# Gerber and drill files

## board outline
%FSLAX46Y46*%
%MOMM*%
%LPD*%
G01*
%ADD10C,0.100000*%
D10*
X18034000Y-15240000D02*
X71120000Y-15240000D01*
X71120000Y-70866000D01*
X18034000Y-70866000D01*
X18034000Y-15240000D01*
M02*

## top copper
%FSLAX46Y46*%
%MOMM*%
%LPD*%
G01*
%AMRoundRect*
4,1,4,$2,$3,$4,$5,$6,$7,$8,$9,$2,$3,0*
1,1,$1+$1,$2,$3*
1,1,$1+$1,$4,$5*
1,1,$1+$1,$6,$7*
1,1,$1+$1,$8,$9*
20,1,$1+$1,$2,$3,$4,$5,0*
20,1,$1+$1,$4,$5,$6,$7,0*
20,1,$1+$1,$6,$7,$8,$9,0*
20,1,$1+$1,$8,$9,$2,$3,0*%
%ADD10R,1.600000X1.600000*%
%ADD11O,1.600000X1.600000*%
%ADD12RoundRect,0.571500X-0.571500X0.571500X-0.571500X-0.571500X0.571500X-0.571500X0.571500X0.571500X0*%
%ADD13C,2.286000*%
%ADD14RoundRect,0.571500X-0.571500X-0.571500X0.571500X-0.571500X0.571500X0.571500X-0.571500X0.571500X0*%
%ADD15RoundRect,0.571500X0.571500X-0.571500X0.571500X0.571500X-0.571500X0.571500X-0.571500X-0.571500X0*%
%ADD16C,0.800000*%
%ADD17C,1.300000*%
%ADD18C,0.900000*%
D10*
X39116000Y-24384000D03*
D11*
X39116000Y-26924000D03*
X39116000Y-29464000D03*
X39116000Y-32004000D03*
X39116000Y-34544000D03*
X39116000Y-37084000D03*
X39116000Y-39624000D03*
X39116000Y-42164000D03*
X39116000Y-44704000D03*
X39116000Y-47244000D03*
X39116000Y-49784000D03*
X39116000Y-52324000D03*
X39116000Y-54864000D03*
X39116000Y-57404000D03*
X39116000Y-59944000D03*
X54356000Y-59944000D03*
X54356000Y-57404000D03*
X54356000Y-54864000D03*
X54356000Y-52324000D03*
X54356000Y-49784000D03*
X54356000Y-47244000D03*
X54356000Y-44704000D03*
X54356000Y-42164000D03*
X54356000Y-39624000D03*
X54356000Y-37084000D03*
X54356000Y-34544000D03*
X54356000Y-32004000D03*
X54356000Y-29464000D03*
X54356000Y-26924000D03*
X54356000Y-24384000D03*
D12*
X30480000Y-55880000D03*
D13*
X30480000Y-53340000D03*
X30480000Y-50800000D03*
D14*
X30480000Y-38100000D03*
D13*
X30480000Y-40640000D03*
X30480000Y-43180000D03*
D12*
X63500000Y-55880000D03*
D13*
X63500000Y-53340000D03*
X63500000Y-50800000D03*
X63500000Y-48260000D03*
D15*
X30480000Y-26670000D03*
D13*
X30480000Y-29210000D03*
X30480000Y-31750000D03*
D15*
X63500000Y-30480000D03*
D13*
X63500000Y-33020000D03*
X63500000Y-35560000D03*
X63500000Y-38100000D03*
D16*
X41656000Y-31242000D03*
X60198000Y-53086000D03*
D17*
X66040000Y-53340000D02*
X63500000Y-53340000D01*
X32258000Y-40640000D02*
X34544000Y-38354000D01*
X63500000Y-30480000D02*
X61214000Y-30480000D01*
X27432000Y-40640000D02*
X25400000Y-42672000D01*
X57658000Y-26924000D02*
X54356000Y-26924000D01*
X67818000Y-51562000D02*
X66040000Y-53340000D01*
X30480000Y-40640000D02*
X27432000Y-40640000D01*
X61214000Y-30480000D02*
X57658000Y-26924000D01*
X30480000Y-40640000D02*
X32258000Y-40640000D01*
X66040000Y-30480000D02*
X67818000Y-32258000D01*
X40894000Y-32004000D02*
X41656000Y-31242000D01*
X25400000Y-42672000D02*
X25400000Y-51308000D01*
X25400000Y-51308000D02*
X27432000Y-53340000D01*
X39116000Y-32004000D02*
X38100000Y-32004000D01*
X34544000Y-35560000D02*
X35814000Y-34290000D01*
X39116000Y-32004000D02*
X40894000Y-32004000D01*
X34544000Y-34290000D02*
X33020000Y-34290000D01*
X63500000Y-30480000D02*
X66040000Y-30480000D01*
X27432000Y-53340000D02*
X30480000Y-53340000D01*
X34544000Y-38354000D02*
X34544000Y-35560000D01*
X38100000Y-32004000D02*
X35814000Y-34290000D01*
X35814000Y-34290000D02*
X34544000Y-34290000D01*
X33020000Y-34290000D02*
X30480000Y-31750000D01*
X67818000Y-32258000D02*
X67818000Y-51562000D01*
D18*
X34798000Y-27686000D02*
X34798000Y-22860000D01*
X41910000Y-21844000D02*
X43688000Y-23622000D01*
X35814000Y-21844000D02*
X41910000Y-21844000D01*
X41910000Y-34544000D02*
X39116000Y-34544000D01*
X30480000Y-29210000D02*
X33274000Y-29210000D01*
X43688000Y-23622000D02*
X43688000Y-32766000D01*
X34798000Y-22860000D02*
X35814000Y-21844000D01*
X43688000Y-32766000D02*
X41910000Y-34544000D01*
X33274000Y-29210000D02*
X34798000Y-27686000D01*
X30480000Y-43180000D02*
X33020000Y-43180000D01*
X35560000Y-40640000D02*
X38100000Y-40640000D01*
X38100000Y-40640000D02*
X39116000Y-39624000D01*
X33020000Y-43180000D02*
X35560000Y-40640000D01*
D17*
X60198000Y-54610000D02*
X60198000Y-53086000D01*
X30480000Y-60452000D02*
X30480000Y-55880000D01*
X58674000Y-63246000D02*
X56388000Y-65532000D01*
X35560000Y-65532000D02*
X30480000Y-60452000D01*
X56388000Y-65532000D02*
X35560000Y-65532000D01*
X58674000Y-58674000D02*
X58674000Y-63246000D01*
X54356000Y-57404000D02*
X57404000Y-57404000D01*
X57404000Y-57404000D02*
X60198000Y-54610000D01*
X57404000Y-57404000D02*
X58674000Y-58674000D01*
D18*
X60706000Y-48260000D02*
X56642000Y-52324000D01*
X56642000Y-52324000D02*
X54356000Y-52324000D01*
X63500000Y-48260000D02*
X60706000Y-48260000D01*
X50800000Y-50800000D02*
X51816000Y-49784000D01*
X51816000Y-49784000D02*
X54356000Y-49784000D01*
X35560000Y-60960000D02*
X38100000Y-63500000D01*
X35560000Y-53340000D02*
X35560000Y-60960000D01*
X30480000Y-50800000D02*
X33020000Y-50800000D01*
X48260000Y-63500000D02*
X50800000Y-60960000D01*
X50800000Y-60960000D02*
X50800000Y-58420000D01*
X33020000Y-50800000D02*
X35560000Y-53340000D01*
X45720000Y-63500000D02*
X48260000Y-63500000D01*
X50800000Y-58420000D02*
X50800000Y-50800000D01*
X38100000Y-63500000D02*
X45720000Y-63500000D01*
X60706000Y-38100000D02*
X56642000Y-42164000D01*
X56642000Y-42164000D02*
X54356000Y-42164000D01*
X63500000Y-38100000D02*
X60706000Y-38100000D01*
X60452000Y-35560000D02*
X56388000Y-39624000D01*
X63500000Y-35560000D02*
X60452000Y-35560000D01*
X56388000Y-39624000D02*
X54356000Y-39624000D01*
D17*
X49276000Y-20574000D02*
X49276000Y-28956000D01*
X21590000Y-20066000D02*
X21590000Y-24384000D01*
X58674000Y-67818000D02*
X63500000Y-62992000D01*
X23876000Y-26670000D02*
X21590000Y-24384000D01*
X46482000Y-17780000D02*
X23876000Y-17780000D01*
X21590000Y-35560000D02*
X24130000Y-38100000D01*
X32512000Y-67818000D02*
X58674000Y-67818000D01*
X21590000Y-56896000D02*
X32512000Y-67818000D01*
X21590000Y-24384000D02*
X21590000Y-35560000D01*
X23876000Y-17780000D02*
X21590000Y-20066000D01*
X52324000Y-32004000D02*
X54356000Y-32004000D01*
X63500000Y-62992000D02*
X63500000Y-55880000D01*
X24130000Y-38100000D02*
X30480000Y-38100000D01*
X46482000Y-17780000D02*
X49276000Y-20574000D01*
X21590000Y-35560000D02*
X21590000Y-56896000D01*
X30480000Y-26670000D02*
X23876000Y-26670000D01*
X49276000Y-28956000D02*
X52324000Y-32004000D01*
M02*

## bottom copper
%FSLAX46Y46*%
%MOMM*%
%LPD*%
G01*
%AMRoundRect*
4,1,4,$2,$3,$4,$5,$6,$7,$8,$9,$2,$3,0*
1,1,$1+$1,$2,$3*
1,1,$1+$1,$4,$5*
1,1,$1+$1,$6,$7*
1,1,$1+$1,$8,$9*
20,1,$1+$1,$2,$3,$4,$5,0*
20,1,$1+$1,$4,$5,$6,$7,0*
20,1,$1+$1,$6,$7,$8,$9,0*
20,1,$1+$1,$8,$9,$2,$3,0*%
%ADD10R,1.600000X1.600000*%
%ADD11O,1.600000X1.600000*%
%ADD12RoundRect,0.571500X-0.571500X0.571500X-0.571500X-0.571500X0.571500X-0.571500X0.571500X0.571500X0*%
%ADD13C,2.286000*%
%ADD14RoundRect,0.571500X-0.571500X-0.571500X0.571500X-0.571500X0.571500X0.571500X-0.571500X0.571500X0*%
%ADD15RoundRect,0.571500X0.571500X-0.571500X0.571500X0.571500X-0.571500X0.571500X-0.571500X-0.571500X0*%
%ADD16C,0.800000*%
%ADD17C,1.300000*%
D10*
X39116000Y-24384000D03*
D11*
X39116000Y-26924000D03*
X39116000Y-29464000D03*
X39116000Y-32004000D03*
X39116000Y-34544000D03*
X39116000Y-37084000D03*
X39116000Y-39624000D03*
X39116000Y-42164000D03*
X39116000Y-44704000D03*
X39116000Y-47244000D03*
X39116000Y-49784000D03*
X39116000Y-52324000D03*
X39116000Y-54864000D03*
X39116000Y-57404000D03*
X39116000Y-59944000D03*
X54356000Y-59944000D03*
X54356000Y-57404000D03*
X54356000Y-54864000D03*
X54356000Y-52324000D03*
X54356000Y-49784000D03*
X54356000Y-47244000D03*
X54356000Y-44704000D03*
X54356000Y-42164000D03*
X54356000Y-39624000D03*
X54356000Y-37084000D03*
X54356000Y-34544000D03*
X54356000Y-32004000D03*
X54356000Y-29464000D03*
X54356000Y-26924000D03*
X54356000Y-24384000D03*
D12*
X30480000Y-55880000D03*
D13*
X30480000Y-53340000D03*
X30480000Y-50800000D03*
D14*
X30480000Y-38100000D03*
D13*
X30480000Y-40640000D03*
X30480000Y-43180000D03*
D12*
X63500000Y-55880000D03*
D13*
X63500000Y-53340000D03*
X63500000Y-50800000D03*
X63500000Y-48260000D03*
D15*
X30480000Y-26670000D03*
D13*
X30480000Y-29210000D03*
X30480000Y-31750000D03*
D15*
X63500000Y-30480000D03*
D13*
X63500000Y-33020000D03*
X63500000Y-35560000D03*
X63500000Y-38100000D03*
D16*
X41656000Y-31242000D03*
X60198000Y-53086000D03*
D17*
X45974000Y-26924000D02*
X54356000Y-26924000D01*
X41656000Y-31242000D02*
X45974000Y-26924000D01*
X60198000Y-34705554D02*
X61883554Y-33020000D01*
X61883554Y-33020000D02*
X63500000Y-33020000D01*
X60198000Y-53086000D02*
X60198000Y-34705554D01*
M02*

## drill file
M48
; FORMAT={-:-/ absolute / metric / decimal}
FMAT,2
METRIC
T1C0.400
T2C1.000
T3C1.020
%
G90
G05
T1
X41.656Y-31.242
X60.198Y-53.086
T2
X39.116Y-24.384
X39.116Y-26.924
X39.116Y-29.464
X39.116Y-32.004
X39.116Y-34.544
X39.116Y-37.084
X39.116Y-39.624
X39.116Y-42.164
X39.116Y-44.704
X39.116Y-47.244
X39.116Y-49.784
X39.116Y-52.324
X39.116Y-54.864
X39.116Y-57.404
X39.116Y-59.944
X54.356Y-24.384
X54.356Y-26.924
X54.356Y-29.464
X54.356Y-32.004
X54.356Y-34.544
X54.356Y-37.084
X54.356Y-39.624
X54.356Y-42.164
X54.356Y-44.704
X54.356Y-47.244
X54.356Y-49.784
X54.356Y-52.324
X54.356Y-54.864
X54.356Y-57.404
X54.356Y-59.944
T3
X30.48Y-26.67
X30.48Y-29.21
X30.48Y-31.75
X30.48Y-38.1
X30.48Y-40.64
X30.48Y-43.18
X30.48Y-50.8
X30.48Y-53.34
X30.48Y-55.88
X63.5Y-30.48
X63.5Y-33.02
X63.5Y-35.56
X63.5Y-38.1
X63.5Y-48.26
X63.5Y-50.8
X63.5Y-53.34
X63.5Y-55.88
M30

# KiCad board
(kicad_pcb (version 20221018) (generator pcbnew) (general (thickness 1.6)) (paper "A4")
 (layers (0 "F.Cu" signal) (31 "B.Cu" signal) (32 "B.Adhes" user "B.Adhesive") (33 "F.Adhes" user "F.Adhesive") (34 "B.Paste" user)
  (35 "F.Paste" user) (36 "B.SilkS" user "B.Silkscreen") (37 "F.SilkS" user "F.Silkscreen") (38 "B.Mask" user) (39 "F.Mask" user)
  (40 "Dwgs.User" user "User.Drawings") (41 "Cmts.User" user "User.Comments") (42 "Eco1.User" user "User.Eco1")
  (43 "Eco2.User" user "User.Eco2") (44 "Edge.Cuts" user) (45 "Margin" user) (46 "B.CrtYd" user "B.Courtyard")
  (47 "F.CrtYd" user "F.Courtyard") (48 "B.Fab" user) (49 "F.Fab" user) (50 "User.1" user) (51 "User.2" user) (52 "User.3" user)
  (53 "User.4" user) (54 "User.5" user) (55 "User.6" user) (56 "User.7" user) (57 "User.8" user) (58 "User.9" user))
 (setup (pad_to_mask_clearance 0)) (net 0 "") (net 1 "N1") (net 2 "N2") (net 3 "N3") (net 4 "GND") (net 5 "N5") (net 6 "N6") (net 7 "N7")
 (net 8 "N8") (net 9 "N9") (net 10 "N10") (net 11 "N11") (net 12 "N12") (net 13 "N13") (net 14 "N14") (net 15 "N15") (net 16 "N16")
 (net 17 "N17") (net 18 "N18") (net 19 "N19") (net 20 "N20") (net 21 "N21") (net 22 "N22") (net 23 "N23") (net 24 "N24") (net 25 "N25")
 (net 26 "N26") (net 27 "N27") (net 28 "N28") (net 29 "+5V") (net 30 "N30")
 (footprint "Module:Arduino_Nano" (layer "F.Cu") (at 39.116 24.384)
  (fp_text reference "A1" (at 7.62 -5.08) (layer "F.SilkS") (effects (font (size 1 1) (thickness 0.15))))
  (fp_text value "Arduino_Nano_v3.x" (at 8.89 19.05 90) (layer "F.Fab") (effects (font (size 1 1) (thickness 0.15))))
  (pad "1" thru_hole rect (at 0 0) (size 1.6 1.6) (drill 1) (layers "*.Cu" "*.Mask") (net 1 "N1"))
  (pad "2" thru_hole oval (at 0 2.54) (size 1.6 1.6) (drill 1) (layers "*.Cu" "*.Mask") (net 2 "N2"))
  (pad "3" thru_hole oval (at 0 5.08) (size 1.6 1.6) (drill 1) (layers "*.Cu" "*.Mask") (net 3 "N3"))
  (pad "4" thru_hole oval (at 0 7.62) (size 1.6 1.6) (drill 1) (layers "*.Cu" "*.Mask") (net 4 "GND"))
  (pad "5" thru_hole oval (at 0 10.16) (size 1.6 1.6) (drill 1) (layers "*.Cu" "*.Mask") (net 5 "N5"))
  (pad "6" thru_hole oval (at 0 12.7) (size 1.6 1.6) (drill 1) (layers "*.Cu" "*.Mask") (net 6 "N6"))
  (pad "7" thru_hole oval (at 0 15.24) (size 1.6 1.6) (drill 1) (layers "*.Cu" "*.Mask") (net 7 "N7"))
  (pad "8" thru_hole oval (at 0 17.78) (size 1.6 1.6) (drill 1) (layers "*.Cu" "*.Mask") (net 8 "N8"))
  (pad "9" thru_hole oval (at 0 20.32) (size 1.6 1.6) (drill 1) (layers "*.Cu" "*.Mask") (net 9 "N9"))
  (pad "10" thru_hole oval (at 0 22.86) (size 1.6 1.6) (drill 1) (layers "*.Cu" "*.Mask") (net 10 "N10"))
  (pad "11" thru_hole oval (at 0 25.4) (size 1.6 1.6) (drill 1) (layers "*.Cu" "*.Mask") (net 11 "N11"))
  (pad "12" thru_hole oval (at 0 27.94) (size 1.6 1.6) (drill 1) (layers "*.Cu" "*.Mask") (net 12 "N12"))
  (pad "13" thru_hole oval (at 0 30.48) (size 1.6 1.6) (drill 1) (layers "*.Cu" "*.Mask") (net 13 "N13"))
  (pad "14" thru_hole oval (at 0 33.02) (size 1.6 1.6) (drill 1) (layers "*.Cu" "*.Mask") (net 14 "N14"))
  (pad "15" thru_hole oval (at 0 35.56) (size 1.6 1.6) (drill 1) (layers "*.Cu" "*.Mask") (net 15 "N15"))
  (pad "16" thru_hole oval (at 15.24 35.56) (size 1.6 1.6) (drill 1) (layers "*.Cu" "*.Mask") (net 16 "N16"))
  (pad "17" thru_hole oval (at 15.24 33.02) (size 1.6 1.6) (drill 1) (layers "*.Cu" "*.Mask") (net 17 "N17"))
  (pad "18" thru_hole oval (at 15.24 30.48) (size 1.6 1.6) (drill 1) (layers "*.Cu" "*.Mask") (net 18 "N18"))
  (pad "19" thru_hole oval (at 15.24 27.94) (size 1.6 1.6) (drill 1) (layers "*.Cu" "*.Mask") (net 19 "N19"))
  (pad "20" thru_hole oval (at 15.24 25.4) (size 1.6 1.6) (drill 1) (layers "*.Cu" "*.Mask") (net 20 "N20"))
  (pad "21" thru_hole oval (at 15.24 22.86) (size 1.6 1.6) (drill 1) (layers "*.Cu" "*.Mask") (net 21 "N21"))
  (pad "22" thru_hole oval (at 15.24 20.32) (size 1.6 1.6) (drill 1) (layers "*.Cu" "*.Mask") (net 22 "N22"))
  (pad "23" thru_hole oval (at 15.24 17.78) (size 1.6 1.6) (drill 1) (layers "*.Cu" "*.Mask") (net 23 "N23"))
  (pad "24" thru_hole oval (at 15.24 15.24) (size 1.6 1.6) (drill 1) (layers "*.Cu" "*.Mask") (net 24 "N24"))
  (pad "25" thru_hole oval (at 15.24 12.7) (size 1.6 1.6) (drill 1) (layers "*.Cu" "*.Mask") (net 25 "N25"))
  (pad "26" thru_hole oval (at 15.24 10.16) (size 1.6 1.6) (drill 1) (layers "*.Cu" "*.Mask") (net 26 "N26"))
  (pad "27" thru_hole oval (at 15.24 7.62) (size 1.6 1.6) (drill 1) (layers "*.Cu" "*.Mask") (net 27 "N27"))
  (pad "28" thru_hole oval (at 15.24 5.08) (size 1.6 1.6) (drill 1) (layers "*.Cu" "*.Mask") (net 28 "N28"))
  (pad "29" thru_hole oval (at 15.24 2.54) (size 1.6 1.6) (drill 1) (layers "*.Cu" "*.Mask") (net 4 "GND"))
  (pad "30" thru_hole oval (at 15.24 0) (size 1.6 1.6) (drill 1) (layers "*.Cu" "*.Mask") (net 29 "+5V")))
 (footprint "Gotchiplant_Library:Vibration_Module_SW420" (layer "F.Cu") (at 30.48 53.34 180)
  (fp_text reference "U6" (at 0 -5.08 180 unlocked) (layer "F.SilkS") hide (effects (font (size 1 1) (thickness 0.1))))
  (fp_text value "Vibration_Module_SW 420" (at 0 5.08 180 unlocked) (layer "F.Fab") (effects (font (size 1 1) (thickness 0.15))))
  (pad "1" thru_hole roundrect (at 0 -2.54 270) (size 2.286 2.286) (drill 1.02) (layers "*.Cu" "*.Mask") (roundrect_rratio 0.25)
   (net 17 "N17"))
  (pad "2" thru_hole circle (at 0 0 270) (size 2.286 2.286) (drill 1.02) (layers "*.Cu" "*.Mask") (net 4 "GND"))
  (pad "3" thru_hole circle (at 0 2.54 270) (size 2.286 2.286) (drill 1.02) (layers "*.Cu" "*.Mask") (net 20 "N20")))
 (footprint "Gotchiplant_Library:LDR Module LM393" (layer "F.Cu") (at 30.48 40.64)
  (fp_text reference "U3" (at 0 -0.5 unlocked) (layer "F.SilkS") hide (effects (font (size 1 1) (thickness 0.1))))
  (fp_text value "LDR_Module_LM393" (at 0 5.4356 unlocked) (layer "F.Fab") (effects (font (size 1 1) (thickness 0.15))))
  (pad "1" thru_hole roundrect (at 0 -2.54) (size 2.286 2.286) (drill 1.02) (layers "*.Cu" "*.Mask") (roundrect_rratio 0.25) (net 27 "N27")
   (thermal_bridge_angle 45))
  (pad "2" thru_hole circle (at 0 0) (size 2.286 2.286) (drill 1.02) (layers "*.Cu" "*.Mask") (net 4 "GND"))
  (pad "3" thru_hole circle (at 0 2.54) (size 2.286 2.286) (drill 1.02) (layers "*.Cu" "*.Mask") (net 7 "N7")))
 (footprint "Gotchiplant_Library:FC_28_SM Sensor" (layer "F.Cu") (at 63.5 52.07 180)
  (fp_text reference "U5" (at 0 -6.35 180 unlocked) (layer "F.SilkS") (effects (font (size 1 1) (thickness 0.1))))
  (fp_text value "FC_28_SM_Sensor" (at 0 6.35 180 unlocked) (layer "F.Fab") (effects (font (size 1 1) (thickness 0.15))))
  (pad "1" thru_hole roundrect (at 0 -3.81 270) (size 2.286 2.286) (drill 1.02) (layers "*.Cu" "*.Mask") (roundrect_rratio 0.25)
   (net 27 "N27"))
  (pad "2" thru_hole circle (at 0 -1.27 270) (size 2.286 2.286) (drill 1.02) (layers "*.Cu" "*.Mask") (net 4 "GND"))
  (pad "3" thru_hole circle (at 0 1.27 270) (size 2.286 2.286) (drill 1.02) (layers "*.Cu" "*.Mask") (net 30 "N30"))
  (pad "4" thru_hole circle (at 0 3.81 270) (size 2.286 2.286) (drill 1.02) (layers "*.Cu" "*.Mask") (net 19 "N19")))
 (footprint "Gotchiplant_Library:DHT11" (layer "F.Cu") (at 30.48 29.21)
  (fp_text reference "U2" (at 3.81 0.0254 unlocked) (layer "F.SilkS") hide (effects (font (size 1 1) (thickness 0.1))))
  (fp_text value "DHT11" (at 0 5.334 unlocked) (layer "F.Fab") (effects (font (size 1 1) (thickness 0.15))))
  (pad "1" thru_hole roundrect (at 0 -2.54 90) (size 2.286 2.286) (drill 1.02) (layers "*.Cu" "*.Mask") (roundrect_rratio 0.25)
   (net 27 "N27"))
  (pad "2" thru_hole circle (at 0 0) (size 2.286 2.286) (drill 1.02) (layers "*.Cu" "*.Mask") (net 5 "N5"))
  (pad "3" thru_hole circle (at 0 2.54) (size 2.286 2.286) (drill 1.02) (layers "*.Cu" "*.Mask") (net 4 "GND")))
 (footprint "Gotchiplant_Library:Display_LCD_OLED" (layer "F.Cu") (at 63.5 34.29)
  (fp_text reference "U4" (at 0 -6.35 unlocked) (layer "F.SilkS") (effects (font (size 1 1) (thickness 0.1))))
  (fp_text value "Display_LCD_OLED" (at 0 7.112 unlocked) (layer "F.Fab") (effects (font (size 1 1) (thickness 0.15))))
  (pad "1" thru_hole roundrect (at 0 -3.81 90) (size 2.286 2.286) (drill 1.02) (layers "*.Cu" "*.Mask") (roundrect_rratio 0.25)
   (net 4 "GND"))
  (pad "2" thru_hole circle (at 0 -1.27 90) (size 2.286 2.286) (drill 1.02) (layers "*.Cu" "*.Mask") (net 17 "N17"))
  (pad "3" thru_hole circle (at 0 1.27 90) (size 2.286 2.286) (drill 1.02) (layers "*.Cu" "*.Mask") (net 24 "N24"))
  (pad "4" thru_hole circle (at 0 3.81 90) (size 2.286 2.286) (drill 1.02) (layers "*.Cu" "*.Mask") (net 23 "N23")))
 (gr_rect (start 18.034 15.24) (end 71.12 70.866) (stroke (width 0.1) (type default)) (fill none) (layer "Edge.Cuts"))
 (segment (start 66.04 53.34) (end 63.5 53.34) (width 1.3) (layer "F.Cu") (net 4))
 (segment (start 32.258 40.64) (end 34.544 38.354) (width 1.3) (layer "F.Cu") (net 4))
 (segment (start 63.5 30.48) (end 61.214 30.48) (width 1.3) (layer "F.Cu") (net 4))
 (segment (start 27.432 40.64) (end 25.4 42.672) (width 1.3) (layer "F.Cu") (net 4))
 (segment (start 57.658 26.924) (end 54.356 26.924) (width 1.3) (layer "F.Cu") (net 4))
 (segment (start 67.818 51.562) (end 66.04 53.34) (width 1.3) (layer "F.Cu") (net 4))
 (segment (start 30.48 40.64) (end 27.432 40.64) (width 1.3) (layer "F.Cu") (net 4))
 (segment (start 61.214 30.48) (end 57.658 26.924) (width 1.3) (layer "F.Cu") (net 4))
 (segment (start 30.48 40.64) (end 32.258 40.64) (width 1.3) (layer "F.Cu") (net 4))
 (segment (start 66.04 30.48) (end 67.818 32.258) (width 1.3) (layer "F.Cu") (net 4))
 (segment (start 40.894 32.004) (end 41.656 31.242) (width 1.3) (layer "F.Cu") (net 4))
 (segment (start 25.4 42.672) (end 25.4 51.308) (width 1.3) (layer "F.Cu") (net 4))
 (segment (start 25.4 51.308) (end 27.432 53.34) (width 1.3) (layer "F.Cu") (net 4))
 (segment (start 39.116 32.004) (end 38.1 32.004) (width 1.3) (layer "F.Cu") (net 4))
 (segment (start 34.544 35.56) (end 35.814 34.29) (width 1.3) (layer "F.Cu") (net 4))
 (segment (start 39.116 32.004) (end 40.894 32.004) (width 1.3) (layer "F.Cu") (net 4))
 (segment (start 34.544 34.29) (end 33.02 34.29) (width 1.3) (layer "F.Cu") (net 4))
 (segment (start 63.5 30.48) (end 66.04 30.48) (width 1.3) (layer "F.Cu") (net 4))
 (segment (start 27.432 53.34) (end 30.48 53.34) (width 1.3) (layer "F.Cu") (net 4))
 (segment (start 34.544 38.354) (end 34.544 35.56) (width 1.3) (layer "F.Cu") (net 4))
 (segment (start 38.1 32.004) (end 35.814 34.29) (width 1.3) (layer "F.Cu") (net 4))
 (segment (start 35.814 34.29) (end 34.544 34.29) (width 1.3) (layer "F.Cu") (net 4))
 (segment (start 33.02 34.29) (end 30.48 31.75) (width 1.3) (layer "F.Cu") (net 4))
 (segment (start 67.818 32.258) (end 67.818 51.562) (width 1.3) (layer "F.Cu") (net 4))
 (via (at 41.656 31.242) (size 0.8) (drill 0.4) (layers "F.Cu" "B.Cu") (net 4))
 (segment (start 45.974 26.924) (end 54.356 26.924) (width 1.3) (layer "B.Cu") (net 4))
 (segment (start 41.656 31.242) (end 45.974 26.924) (width 1.3) (layer "B.Cu") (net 4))
 (segment (start 34.798 27.686) (end 34.798 22.86) (width 0.9) (layer "F.Cu") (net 5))
 (segment (start 41.91 21.844) (end 43.688 23.622) (width 0.9) (layer "F.Cu") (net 5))
 (segment (start 35.814 21.844) (end 41.91 21.844) (width 0.9) (layer "F.Cu") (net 5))
 (segment (start 41.91 34.544) (end 39.116 34.544) (width 0.9) (layer "F.Cu") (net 5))
 (segment (start 30.48 29.21) (end 33.274 29.21) (width 0.9) (layer "F.Cu") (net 5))
 (segment (start 43.688 23.622) (end 43.688 32.766) (width 0.9) (layer "F.Cu") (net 5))
 (segment (start 34.798 22.86) (end 35.814 21.844) (width 0.9) (layer "F.Cu") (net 5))
 (segment (start 43.688 32.766) (end 41.91 34.544) (width 0.9) (layer "F.Cu") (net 5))
 (segment (start 33.274 29.21) (end 34.798 27.686) (width 0.9) (layer "F.Cu") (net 5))
 (segment (start 30.48 43.18) (end 33.02 43.18) (width 0.9) (layer "F.Cu") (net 7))
 (segment (start 35.56 40.64) (end 38.1 40.64) (width 0.9) (layer "F.Cu") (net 7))
 (segment (start 38.1 40.64) (end 39.116 39.624) (width 0.9) (layer "F.Cu") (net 7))
 (segment (start 33.02 43.18) (end 35.56 40.64) (width 0.9) (layer "F.Cu") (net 7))
 (segment (start 60.198 54.61) (end 60.198 53.086) (width 1.3) (layer "F.Cu") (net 17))
 (segment (start 30.48 60.452) (end 30.48 55.88) (width 1.3) (layer "F.Cu") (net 17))
 (segment (start 58.674 63.246) (end 56.388 65.532) (width 1.3) (layer "F.Cu") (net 17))
 (segment (start 35.56 65.532) (end 30.48 60.452) (width 1.3) (layer "F.Cu") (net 17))
 (segment (start 56.388 65.532) (end 35.56 65.532) (width 1.3) (layer "F.Cu") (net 17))
 (segment (start 58.674 58.674) (end 58.674 63.246) (width 1.3) (layer "F.Cu") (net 17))
 (segment (start 54.356 57.404) (end 57.404 57.404) (width 1.3) (layer "F.Cu") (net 17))
 (segment (start 57.404 57.404) (end 60.198 54.61) (width 1.3) (layer "F.Cu") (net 17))
 (segment (start 57.404 57.404) (end 58.674 58.674) (width 1.3) (layer "F.Cu") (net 17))
 (via (at 60.198 53.086) (size 0.8) (drill 0.4) (layers "F.Cu" "B.Cu") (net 17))
 (segment (start 60.198 34.705554) (end 61.883554 33.02) (width 1.3) (layer "B.Cu") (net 17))
 (segment (start 61.883554 33.02) (end 63.5 33.02) (width 1.3) (layer "B.Cu") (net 17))
 (segment (start 60.198 53.086) (end 60.198 34.705554) (width 1.3) (layer "B.Cu") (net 17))
 (segment (start 60.706 48.26) (end 56.642 52.324) (width 0.9) (layer "F.Cu") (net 19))
 (segment (start 56.642 52.324) (end 54.356 52.324) (width 0.9) (layer "F.Cu") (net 19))
 (segment (start 63.5 48.26) (end 60.706 48.26) (width 0.9) (layer "F.Cu") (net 19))
 (segment (start 50.8 50.8) (end 51.816 49.784) (width 0.9) (layer "F.Cu") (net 20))
 (segment (start 51.816 49.784) (end 54.356 49.784) (width 0.9) (layer "F.Cu") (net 20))
 (segment (start 35.56 60.96) (end 38.1 63.5) (width 0.9) (layer "F.Cu") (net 20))
 (segment (start 35.56 53.34) (end 35.56 60.96) (width 0.9) (layer "F.Cu") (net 20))
 (segment (start 30.48 50.8) (end 33.02 50.8) (width 0.9) (layer "F.Cu") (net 20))
 (segment (start 48.26 63.5) (end 50.8 60.96) (width 0.9) (layer "F.Cu") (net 20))
 (segment (start 50.8 60.96) (end 50.8 58.42) (width 0.9) (layer "F.Cu") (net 20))
 (segment (start 33.02 50.8) (end 35.56 53.34) (width 0.9) (layer "F.Cu") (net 20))
 (segment (start 45.72 63.5) (end 48.26 63.5) (width 0.9) (layer "F.Cu") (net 20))
 (segment (start 50.8 58.42) (end 50.8 50.8) (width 0.9) (layer "F.Cu") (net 20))
 (segment (start 38.1 63.5) (end 45.72 63.5) (width 0.9) (layer "F.Cu") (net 20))
 (segment (start 60.706 38.1) (end 56.642 42.164) (width 0.9) (layer "F.Cu") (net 23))
 (segment (start 56.642 42.164) (end 54.356 42.164) (width 0.9) (layer "F.Cu") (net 23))
 (segment (start 63.5 38.1) (end 60.706 38.1) (width 0.9) (layer "F.Cu") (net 23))
 (segment (start 60.452 35.56) (end 56.388 39.624) (width 0.9) (layer "F.Cu") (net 24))
 (segment (start 63.5 35.56) (end 60.452 35.56) (width 0.9) (layer "F.Cu") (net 24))
 (segment (start 56.388 39.624) (end 54.356 39.624) (width 0.9) (layer "F.Cu") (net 24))
 (segment (start 49.276 20.574) (end 49.276 28.956) (width 1.3) (layer "F.Cu") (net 27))
 (segment (start 21.59 20.066) (end 21.59 24.384) (width 1.3) (layer "F.Cu") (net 27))
 (segment (start 58.674 67.818) (end 63.5 62.992) (width 1.3) (layer "F.Cu") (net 27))
 (segment (start 23.876 26.67) (end 21.59 24.384) (width 1.3) (layer "F.Cu") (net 27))
 (segment (start 46.482 17.78) (end 23.876 17.78) (width 1.3) (layer "F.Cu") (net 27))
 (segment (start 21.59 35.56) (end 24.13 38.1) (width 1.3) (layer "F.Cu") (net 27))
 (segment (start 32.512 67.818) (end 58.674 67.818) (width 1.3) (layer "F.Cu") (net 27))
 (segment (start 21.59 56.896) (end 32.512 67.818) (width 1.3) (layer "F.Cu") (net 27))
 (segment (start 21.59 24.384) (end 21.59 35.56) (width 1.3) (layer "F.Cu") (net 27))
 (segment (start 23.876 17.78) (end 21.59 20.066) (width 1.3) (layer "F.Cu") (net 27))
 (segment (start 52.324 32.004) (end 54.356 32.004) (width 1.3) (layer "F.Cu") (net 27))
 (segment (start 63.5 62.992) (end 63.5 55.88) (width 1.3) (layer "F.Cu") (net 27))
 (segment (start 24.13 38.1) (end 30.48 38.1) (width 1.3) (layer "F.Cu") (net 27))
 (segment (start 46.482 17.78) (end 49.276 20.574) (width 1.3) (layer "F.Cu") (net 27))
 (segment (start 21.59 35.56) (end 21.59 56.896) (width 1.3) (layer "F.Cu") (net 27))
 (segment (start 30.48 26.67) (end 23.876 26.67) (width 1.3) (layer "F.Cu") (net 27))
 (segment (start 49.276 28.956) (end 52.324 32.004) (width 1.3) (layer "F.Cu") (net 27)))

